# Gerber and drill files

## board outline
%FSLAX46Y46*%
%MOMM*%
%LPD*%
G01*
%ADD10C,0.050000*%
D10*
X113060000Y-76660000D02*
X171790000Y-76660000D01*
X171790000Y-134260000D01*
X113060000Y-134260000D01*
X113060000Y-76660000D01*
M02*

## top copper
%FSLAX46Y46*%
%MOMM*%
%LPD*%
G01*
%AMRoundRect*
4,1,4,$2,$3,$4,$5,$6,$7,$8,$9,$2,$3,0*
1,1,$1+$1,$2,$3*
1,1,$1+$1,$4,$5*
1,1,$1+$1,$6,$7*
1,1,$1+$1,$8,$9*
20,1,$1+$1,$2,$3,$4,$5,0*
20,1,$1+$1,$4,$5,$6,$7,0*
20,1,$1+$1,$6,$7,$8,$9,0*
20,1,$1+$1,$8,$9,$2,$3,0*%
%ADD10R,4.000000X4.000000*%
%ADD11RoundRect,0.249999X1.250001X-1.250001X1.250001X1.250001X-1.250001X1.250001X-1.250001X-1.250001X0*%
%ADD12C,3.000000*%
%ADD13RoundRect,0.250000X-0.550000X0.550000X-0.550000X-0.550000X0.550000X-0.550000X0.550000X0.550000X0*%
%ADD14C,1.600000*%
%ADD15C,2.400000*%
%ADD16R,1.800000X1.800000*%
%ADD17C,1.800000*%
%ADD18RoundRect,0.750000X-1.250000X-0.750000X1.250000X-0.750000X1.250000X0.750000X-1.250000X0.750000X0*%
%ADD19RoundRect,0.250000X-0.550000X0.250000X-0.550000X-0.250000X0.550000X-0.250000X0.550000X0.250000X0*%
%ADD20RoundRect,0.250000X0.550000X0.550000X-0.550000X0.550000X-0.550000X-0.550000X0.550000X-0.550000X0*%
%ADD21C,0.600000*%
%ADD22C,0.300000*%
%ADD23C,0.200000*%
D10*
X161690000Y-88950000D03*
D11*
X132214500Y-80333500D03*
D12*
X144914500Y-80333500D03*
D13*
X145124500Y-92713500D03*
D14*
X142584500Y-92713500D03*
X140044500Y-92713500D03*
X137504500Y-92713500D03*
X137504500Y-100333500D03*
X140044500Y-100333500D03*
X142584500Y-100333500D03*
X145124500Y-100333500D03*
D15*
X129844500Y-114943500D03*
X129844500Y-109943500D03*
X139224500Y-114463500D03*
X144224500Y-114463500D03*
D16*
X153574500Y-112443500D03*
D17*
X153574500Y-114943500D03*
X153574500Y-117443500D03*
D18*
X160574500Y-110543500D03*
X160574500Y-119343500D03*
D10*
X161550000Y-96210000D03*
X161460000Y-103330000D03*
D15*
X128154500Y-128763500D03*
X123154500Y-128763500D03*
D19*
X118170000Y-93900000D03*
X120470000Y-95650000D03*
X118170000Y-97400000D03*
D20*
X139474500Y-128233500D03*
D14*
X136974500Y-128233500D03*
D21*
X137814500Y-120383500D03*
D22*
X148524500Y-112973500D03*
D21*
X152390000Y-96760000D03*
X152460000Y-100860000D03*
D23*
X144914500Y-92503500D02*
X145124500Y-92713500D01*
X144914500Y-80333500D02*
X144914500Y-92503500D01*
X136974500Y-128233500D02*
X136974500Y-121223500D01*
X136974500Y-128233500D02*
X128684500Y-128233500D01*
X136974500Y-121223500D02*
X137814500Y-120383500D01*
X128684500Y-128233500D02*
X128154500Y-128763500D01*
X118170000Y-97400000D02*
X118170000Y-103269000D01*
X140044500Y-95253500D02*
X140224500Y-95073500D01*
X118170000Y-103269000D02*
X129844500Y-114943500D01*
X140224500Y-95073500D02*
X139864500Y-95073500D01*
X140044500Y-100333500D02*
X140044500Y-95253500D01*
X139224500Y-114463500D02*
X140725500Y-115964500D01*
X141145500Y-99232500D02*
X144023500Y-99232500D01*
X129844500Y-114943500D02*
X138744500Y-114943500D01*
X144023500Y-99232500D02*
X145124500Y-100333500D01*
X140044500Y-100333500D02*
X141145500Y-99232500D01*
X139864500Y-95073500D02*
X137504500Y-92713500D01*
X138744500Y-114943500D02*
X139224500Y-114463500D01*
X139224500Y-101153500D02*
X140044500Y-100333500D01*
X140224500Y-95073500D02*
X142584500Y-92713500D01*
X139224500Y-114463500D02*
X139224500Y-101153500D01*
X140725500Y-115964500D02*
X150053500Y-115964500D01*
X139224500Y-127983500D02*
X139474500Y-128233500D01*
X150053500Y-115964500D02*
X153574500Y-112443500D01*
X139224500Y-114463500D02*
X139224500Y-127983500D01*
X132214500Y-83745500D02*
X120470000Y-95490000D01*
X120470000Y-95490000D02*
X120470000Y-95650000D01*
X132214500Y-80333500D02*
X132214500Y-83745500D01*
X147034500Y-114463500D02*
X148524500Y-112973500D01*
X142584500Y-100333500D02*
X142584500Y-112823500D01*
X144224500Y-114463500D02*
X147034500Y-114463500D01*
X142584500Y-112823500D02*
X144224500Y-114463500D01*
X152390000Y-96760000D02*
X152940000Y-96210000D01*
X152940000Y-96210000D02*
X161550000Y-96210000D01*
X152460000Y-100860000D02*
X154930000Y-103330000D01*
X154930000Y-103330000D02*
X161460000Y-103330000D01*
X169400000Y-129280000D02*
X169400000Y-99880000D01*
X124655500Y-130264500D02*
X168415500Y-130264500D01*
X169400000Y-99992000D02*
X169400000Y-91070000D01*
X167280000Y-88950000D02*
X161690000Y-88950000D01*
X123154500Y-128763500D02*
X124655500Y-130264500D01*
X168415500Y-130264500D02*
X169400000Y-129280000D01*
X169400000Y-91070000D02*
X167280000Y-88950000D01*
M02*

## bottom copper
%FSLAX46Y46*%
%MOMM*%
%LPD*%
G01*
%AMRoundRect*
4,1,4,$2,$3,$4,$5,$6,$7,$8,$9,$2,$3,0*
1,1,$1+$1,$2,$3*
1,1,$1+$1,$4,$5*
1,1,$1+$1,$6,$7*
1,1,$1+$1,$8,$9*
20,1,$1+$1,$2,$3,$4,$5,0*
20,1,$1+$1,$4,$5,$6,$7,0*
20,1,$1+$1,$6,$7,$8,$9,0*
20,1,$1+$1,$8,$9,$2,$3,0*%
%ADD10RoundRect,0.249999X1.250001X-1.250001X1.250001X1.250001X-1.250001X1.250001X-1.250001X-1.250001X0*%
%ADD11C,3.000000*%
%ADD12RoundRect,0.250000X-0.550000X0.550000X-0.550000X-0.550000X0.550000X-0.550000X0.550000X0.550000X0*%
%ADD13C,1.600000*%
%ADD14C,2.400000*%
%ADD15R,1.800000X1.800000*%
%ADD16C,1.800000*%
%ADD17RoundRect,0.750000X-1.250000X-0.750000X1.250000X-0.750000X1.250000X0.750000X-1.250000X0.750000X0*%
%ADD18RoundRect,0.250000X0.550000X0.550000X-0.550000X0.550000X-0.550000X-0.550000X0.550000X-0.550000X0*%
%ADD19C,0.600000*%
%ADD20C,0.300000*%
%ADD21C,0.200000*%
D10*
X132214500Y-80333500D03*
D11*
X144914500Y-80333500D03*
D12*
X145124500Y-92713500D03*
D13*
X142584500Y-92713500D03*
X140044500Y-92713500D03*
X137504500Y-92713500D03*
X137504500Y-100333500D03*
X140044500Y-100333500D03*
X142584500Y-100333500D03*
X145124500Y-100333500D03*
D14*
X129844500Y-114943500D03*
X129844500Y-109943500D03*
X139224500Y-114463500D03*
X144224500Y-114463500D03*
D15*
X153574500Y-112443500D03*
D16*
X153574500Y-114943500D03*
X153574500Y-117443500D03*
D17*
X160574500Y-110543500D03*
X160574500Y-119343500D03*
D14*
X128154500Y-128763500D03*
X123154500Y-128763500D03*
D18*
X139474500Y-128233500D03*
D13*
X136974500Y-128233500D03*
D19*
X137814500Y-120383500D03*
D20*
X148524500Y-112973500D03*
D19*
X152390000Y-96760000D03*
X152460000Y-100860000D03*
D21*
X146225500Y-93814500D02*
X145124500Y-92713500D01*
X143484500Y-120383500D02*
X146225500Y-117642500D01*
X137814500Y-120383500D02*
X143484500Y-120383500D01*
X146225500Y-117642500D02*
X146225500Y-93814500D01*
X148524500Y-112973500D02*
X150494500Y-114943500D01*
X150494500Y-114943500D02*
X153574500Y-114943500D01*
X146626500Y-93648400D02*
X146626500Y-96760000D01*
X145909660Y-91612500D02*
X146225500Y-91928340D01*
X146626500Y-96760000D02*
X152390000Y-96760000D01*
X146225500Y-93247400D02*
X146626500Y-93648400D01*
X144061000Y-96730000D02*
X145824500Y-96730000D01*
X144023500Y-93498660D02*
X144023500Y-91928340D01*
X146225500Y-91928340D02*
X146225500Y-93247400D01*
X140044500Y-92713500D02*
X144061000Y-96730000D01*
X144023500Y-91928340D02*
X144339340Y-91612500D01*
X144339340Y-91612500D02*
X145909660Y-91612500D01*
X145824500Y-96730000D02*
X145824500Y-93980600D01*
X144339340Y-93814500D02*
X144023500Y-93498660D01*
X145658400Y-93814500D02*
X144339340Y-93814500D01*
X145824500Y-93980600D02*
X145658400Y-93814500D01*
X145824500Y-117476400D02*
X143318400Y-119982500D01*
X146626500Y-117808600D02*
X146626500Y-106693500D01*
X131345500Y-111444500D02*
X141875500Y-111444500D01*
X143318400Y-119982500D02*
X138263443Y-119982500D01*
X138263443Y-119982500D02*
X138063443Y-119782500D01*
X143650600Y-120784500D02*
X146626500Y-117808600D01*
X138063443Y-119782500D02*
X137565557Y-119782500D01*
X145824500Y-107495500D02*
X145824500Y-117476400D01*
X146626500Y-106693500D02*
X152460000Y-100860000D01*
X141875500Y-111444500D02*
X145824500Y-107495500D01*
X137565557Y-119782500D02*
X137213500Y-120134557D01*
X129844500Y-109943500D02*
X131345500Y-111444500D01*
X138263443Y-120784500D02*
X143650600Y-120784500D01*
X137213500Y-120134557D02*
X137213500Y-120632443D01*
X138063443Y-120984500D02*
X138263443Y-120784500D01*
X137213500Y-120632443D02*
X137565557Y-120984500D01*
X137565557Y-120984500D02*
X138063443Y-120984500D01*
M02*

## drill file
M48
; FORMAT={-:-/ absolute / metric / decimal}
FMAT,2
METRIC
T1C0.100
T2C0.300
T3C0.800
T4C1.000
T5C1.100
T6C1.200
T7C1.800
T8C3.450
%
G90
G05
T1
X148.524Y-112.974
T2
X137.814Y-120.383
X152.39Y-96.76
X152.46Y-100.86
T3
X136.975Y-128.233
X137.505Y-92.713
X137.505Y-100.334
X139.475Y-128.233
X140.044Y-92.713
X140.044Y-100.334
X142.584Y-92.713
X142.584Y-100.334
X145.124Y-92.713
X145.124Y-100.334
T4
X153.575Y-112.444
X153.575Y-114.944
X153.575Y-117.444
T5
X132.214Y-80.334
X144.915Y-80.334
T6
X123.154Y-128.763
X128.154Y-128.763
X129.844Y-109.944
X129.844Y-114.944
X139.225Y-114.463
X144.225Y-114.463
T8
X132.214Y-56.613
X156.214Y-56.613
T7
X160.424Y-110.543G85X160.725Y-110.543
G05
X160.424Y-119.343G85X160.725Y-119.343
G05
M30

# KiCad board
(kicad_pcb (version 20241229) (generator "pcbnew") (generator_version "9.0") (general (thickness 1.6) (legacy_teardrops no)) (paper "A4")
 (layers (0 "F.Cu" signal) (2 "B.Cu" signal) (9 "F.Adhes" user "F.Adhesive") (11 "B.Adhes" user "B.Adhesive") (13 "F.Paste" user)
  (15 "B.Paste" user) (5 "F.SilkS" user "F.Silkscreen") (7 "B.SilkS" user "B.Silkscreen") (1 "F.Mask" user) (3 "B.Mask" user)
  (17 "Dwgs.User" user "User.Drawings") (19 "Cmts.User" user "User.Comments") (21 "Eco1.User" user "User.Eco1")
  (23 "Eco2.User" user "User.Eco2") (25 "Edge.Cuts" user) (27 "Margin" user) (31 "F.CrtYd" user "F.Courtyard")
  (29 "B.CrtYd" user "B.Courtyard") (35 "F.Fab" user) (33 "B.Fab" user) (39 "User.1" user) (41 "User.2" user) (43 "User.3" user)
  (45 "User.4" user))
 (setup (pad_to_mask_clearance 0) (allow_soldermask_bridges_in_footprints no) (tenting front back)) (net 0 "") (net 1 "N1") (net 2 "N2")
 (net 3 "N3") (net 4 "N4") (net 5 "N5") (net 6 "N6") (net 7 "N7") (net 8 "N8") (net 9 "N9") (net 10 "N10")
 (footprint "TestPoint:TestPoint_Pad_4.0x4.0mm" (layer "F.Cu") (at 161.69 88.95)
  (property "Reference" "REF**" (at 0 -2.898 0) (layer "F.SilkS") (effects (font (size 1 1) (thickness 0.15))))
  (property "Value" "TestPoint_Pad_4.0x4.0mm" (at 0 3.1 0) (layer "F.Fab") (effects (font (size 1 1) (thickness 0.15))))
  (pad "1" smd rect (at 0 0) (size 4 4) (layers "F.Cu" "F.Mask") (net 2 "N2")))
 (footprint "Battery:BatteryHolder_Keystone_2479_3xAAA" (layer "F.Cu") (at 132.2145 80.3335 90)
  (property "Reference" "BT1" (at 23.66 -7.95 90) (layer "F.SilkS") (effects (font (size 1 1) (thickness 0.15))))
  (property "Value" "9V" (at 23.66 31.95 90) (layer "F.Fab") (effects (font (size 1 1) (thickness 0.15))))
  (pad "" np_thru_hole circle (at 23.72 0 90) (size 3.45 3.45) (drill 3.45) (layers "*.Cu" "*.Mask"))
  (pad "" np_thru_hole circle (at 23.72 24 90) (size 3.45 3.45) (drill 3.45) (layers "*.Cu" "*.Mask"))
  (pad "1" thru_hole roundrect (at 0 0 90) (size 3 3) (drill 1.1) (layers "*.Cu" "*.Mask") (remove_unused_layers no)
   (roundrect_rratio 0.083333) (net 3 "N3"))
  (pad "2" thru_hole circle (at 0 12.7 90) (size 3 3) (drill 1.1) (layers "*.Cu" "*.Mask") (remove_unused_layers no) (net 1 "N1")))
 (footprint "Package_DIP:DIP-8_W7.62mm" (layer "F.Cu") (at 145.1245 92.7135 -90)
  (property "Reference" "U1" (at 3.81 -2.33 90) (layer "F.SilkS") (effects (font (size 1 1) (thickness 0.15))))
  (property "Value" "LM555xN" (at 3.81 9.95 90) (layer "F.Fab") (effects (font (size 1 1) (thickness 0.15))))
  (pad "1" thru_hole roundrect (at 0 0 270) (size 1.6 1.6) (drill 0.8) (layers "*.Cu" "*.Mask") (remove_unused_layers no)
   (roundrect_rratio 0.15625) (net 1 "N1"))
  (pad "2" thru_hole circle (at 0 2.54 270) (size 1.6 1.6) (drill 0.8) (layers "*.Cu" "*.Mask") (remove_unused_layers no) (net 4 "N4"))
  (pad "3" thru_hole circle (at 0 5.08 270) (size 1.6 1.6) (drill 0.8) (layers "*.Cu" "*.Mask") (remove_unused_layers no) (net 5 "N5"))
  (pad "4" thru_hole circle (at 0 7.62 270) (size 1.6 1.6) (drill 0.8) (layers "*.Cu" "*.Mask") (remove_unused_layers no) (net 4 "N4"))
  (pad "5" thru_hole circle (at 7.62 7.62 270) (size 1.6 1.6) (drill 0.8) (layers "*.Cu" "*.Mask") (remove_unused_layers no) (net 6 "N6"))
  (pad "6" thru_hole circle (at 7.62 5.08 270) (size 1.6 1.6) (drill 0.8) (layers "*.Cu" "*.Mask") (remove_unused_layers no) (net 4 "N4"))
  (pad "7" thru_hole circle (at 7.62 2.54 270) (size 1.6 1.6) (drill 0.8) (layers "*.Cu" "*.Mask") (remove_unused_layers no) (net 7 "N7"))
  (pad "8" thru_hole circle (at 7.62 0 270) (size 1.6 1.6) (drill 0.8) (layers "*.Cu" "*.Mask") (remove_unused_layers no) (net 4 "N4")))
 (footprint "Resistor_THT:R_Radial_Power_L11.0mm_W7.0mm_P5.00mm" (layer "F.Cu") (at 129.8445 114.9435 90)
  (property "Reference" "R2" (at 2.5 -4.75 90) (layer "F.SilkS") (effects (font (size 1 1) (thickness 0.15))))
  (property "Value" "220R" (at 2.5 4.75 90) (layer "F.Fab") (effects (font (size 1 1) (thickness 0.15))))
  (pad "1" thru_hole circle (at 0 0 90) (size 2.4 2.4) (drill 1.2) (layers "*.Cu" "*.Mask") (remove_unused_layers no) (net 4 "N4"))
  (pad "2" thru_hole circle (at 5 0 90) (size 2.4 2.4) (drill 1.2) (layers "*.Cu" "*.Mask") (remove_unused_layers no) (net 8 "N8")))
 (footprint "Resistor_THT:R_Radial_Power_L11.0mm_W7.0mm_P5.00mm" (layer "F.Cu") (at 139.2245 114.4635)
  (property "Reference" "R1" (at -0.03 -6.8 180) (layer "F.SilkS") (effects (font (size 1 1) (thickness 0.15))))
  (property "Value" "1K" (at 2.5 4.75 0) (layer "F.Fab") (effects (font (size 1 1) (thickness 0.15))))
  (pad "1" thru_hole circle (at 0 0) (size 2.4 2.4) (drill 1.2) (layers "*.Cu" "*.Mask") (remove_unused_layers no) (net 4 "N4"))
  (pad "2" thru_hole circle (at 5 0) (size 2.4 2.4) (drill 1.2) (layers "*.Cu" "*.Mask") (remove_unused_layers no) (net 7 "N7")))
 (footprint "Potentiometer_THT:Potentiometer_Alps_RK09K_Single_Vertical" (layer "F.Cu") (at 153.5745 112.4435)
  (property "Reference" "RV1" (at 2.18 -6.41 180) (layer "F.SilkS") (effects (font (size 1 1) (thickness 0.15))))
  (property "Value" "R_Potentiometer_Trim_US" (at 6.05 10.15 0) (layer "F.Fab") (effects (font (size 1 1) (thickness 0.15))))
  (pad "1" thru_hole rect (at 0 0) (size 1.8 1.8) (drill 1) (layers "*.Cu" "*.Mask") (remove_unused_layers no) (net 4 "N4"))
  (pad "2" thru_hole circle (at 0 2.5) (size 1.8 1.8) (drill 1) (layers "*.Cu" "*.Mask") (remove_unused_layers no) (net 7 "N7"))
  (pad "3" thru_hole circle (at 0 5) (size 1.8 1.8) (drill 1) (layers "*.Cu" "*.Mask") (remove_unused_layers no) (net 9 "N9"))
  (pad "MP" thru_hole roundrect (at 7 -1.9) (size 4 3) (drill oval 2.1 1.8) (layers "*.Cu" "*.Mask") (remove_unused_layers no)
   (roundrect_rratio 0.25))
  (pad "MP" thru_hole roundrect (at 7 6.9) (size 4 3) (drill oval 2.1 1.8) (layers "*.Cu" "*.Mask") (remove_unused_layers no)
   (roundrect_rratio 0.25)))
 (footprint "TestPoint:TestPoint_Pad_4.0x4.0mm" (layer "F.Cu") (at 161.55 96.21)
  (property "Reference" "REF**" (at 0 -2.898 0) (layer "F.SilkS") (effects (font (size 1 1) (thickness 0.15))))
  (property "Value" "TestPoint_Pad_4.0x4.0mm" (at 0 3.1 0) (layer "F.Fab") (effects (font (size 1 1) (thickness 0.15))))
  (pad "1" smd rect (at 0 0) (size 4 4) (layers "F.Cu" "F.Mask") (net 5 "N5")))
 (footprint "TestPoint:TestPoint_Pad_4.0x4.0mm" (layer "F.Cu") (at 161.46 103.33)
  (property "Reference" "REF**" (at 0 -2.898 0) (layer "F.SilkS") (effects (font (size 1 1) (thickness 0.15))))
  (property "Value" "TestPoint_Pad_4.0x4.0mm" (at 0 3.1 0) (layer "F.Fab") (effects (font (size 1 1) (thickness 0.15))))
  (pad "1" smd rect (at 0 0) (size 4 4) (layers "F.Cu" "F.Mask") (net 8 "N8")))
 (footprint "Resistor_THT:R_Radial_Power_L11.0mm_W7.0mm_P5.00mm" (layer "F.Cu") (at 128.1545 128.7635 180)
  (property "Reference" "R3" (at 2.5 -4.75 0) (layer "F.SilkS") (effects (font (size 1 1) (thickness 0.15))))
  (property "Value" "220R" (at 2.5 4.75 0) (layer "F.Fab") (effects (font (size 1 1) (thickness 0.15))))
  (pad "1" thru_hole circle (at 0 0 180) (size 2.4 2.4) (drill 1.2) (layers "*.Cu" "*.Mask") (remove_unused_layers no) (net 1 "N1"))
  (pad "2" thru_hole circle (at 5 0 180) (size 2.4 2.4) (drill 1.2) (layers "*.Cu" "*.Mask") (remove_unused_layers no) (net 2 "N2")))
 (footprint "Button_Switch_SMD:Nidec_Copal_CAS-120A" (layer "F.Cu") (at 119.32 95.65)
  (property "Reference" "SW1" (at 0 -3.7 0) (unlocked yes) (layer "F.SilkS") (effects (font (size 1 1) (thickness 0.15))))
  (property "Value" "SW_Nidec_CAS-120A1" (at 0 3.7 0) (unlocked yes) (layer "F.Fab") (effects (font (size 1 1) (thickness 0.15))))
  (pad "1" smd roundrect (at -1.15 -1.75 270) (size 1 1.6) (layers "F.Cu" "F.Mask" "F.Paste") (roundrect_rratio 0.25) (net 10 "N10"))
  (pad "2" smd roundrect (at 1.15 0 270) (size 1 1.6) (layers "F.Cu" "F.Mask" "F.Paste") (roundrect_rratio 0.25) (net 3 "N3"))
  (pad "3" smd roundrect (at -1.15 1.75 270) (size 1 1.6) (layers "F.Cu" "F.Mask" "F.Paste") (roundrect_rratio 0.25) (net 4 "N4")))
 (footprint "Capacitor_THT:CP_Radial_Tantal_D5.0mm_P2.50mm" (layer "F.Cu") (at 139.4745 128.2335 180)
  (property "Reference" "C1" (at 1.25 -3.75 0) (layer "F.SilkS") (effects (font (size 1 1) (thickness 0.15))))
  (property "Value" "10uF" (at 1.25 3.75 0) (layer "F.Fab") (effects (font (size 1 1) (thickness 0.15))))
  (pad "1" thru_hole roundrect (at 0 0 180) (size 1.6 1.6) (drill 0.8) (layers "*.Cu" "*.Mask") (remove_unused_layers no)
   (roundrect_rratio 0.15625) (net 4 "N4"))
  (pad "2" thru_hole circle (at 2.5 0 180) (size 1.6 1.6) (drill 0.8) (layers "*.Cu" "*.Mask") (remove_unused_layers no) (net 1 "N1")))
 (gr_rect (start 113.06 76.66) (end 171.79 134.26) (stroke (width 0.05) (type default)) (fill no) (layer "Edge.Cuts"))
 (segment (start 144.9145 92.5035) (end 145.1245 92.7135) (width 0.2) (layer "F.Cu") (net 1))
 (segment (start 144.9145 80.3335) (end 144.9145 92.5035) (width 0.2) (layer "F.Cu") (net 1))
 (segment (start 136.9745 128.2335) (end 136.9745 121.2235) (width 0.2) (layer "F.Cu") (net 1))
 (segment (start 136.9745 128.2335) (end 128.6845 128.2335) (width 0.2) (layer "F.Cu") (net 1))
 (segment (start 136.9745 121.2235) (end 137.8145 120.3835) (width 0.2) (layer "F.Cu") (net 1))
 (segment (start 128.6845 128.2335) (end 128.1545 128.7635) (width 0.2) (layer "F.Cu") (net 1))
 (via (at 137.8145 120.3835) (size 0.6) (drill 0.3) (layers "F.Cu" "B.Cu") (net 1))
 (segment (start 146.2255 93.8145) (end 145.1245 92.7135) (width 0.2) (layer "B.Cu") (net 1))
 (segment (start 143.4845 120.3835) (end 146.2255 117.6425) (width 0.2) (layer "B.Cu") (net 1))
 (segment (start 137.8145 120.3835) (end 143.4845 120.3835) (width 0.2) (layer "B.Cu") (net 1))
 (segment (start 146.2255 117.6425) (end 146.2255 93.8145) (width 0.2) (layer "B.Cu") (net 1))
 (segment (start 118.17 97.4) (end 118.17 103.269) (width 0.2) (layer "F.Cu") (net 4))
 (segment (start 140.0445 95.2535) (end 140.2245 95.0735) (width 0.2) (layer "F.Cu") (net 4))
 (segment (start 118.17 103.269) (end 129.8445 114.9435) (width 0.2) (layer "F.Cu") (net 4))
 (segment (start 140.2245 95.0735) (end 139.8645 95.0735) (width 0.2) (layer "F.Cu") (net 4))
 (segment (start 140.0445 100.3335) (end 140.0445 95.2535) (width 0.2) (layer "F.Cu") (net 4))
 (segment (start 139.2245 114.4635) (end 140.7255 115.9645) (width 0.2) (layer "F.Cu") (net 4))
 (segment (start 141.1455 99.2325) (end 144.0235 99.2325) (width 0.2) (layer "F.Cu") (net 4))
 (segment (start 129.8445 114.9435) (end 138.7445 114.9435) (width 0.2) (layer "F.Cu") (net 4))
 (segment (start 144.0235 99.2325) (end 145.1245 100.3335) (width 0.2) (layer "F.Cu") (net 4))
 (segment (start 140.0445 100.3335) (end 141.1455 99.2325) (width 0.2) (layer "F.Cu") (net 4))
 (segment (start 139.8645 95.0735) (end 137.5045 92.7135) (width 0.2) (layer "F.Cu") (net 4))
 (segment (start 138.7445 114.9435) (end 139.2245 114.4635) (width 0.2) (layer "F.Cu") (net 4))
 (segment (start 139.2245 101.1535) (end 140.0445 100.3335) (width 0.2) (layer "F.Cu") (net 4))
 (segment (start 140.2245 95.0735) (end 142.5845 92.7135) (width 0.2) (layer "F.Cu") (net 4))
 (segment (start 139.2245 114.4635) (end 139.2245 101.1535) (width 0.2) (layer "F.Cu") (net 4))
 (segment (start 140.7255 115.9645) (end 150.0535 115.9645) (width 0.2) (layer "F.Cu") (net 4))
 (segment (start 139.2245 127.9835) (end 139.4745 128.2335) (width 0.2) (layer "F.Cu") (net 4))
 (segment (start 150.0535 115.9645) (end 153.5745 112.4435) (width 0.2) (layer "F.Cu") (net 4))
 (segment (start 139.2245 114.4635) (end 139.2245 127.9835) (width 0.2) (layer "F.Cu") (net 4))
 (segment (start 132.2145 83.7455) (end 120.47 95.49) (width 0.2) (layer "F.Cu") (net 3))
 (segment (start 120.47 95.49) (end 120.47 95.65) (width 0.2) (layer "F.Cu") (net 3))
 (segment (start 132.2145 80.3335) (end 132.2145 83.7455) (width 0.2) (layer "F.Cu") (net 3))
 (segment (start 147.0345 114.4635) (end 148.5245 112.9735) (width 0.2) (layer "F.Cu") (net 7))
 (segment (start 142.5845 100.3335) (end 142.5845 112.8235) (width 0.2) (layer "F.Cu") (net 7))
 (segment (start 144.2245 114.4635) (end 147.0345 114.4635) (width 0.2) (layer "F.Cu") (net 7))
 (segment (start 142.5845 112.8235) (end 144.2245 114.4635) (width 0.2) (layer "F.Cu") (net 7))
 (via micro (at 148.5245 112.9735) (size 0.3) (drill 0.1) (layers "F.Cu" "B.Cu") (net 7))
 (segment (start 148.5245 112.9735) (end 150.4945 114.9435) (width 0.2) (layer "B.Cu") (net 7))
 (segment (start 150.4945 114.9435) (end 153.5745 114.9435) (width 0.2) (layer "B.Cu") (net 7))
 (segment (start 152.39 96.76) (end 152.94 96.21) (width 0.2) (layer "F.Cu") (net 5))
 (segment (start 152.94 96.21) (end 161.55 96.21) (width 0.2) (layer "F.Cu") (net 5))
 (via (at 152.39 96.76) (size 0.6) (drill 0.3) (layers "F.Cu" "B.Cu") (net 5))
 (segment (start 146.6265 93.6484) (end 146.6265 96.76) (width 0.2) (layer "B.Cu") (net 5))
 (segment (start 145.90966 91.6125) (end 146.2255 91.92834) (width 0.2) (layer "B.Cu") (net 5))
 (segment (start 146.6265 96.76) (end 152.39 96.76) (width 0.2) (layer "B.Cu") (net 5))
 (segment (start 146.2255 93.2474) (end 146.6265 93.6484) (width 0.2) (layer "B.Cu") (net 5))
 (segment (start 144.061 96.73) (end 145.8245 96.73) (width 0.2) (layer "B.Cu") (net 5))
 (segment (start 144.0235 93.49866) (end 144.0235 91.92834) (width 0.2) (layer "B.Cu") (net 5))
 (segment (start 146.2255 91.92834) (end 146.2255 93.2474) (width 0.2) (layer "B.Cu") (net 5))
 (segment (start 140.0445 92.7135) (end 144.061 96.73) (width 0.2) (layer "B.Cu") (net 5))
 (segment (start 144.0235 91.92834) (end 144.33934 91.6125) (width 0.2) (layer "B.Cu") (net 5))
 (segment (start 144.33934 91.6125) (end 145.90966 91.6125) (width 0.2) (layer "B.Cu") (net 5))
 (segment (start 145.8245 96.73) (end 145.8245 93.9806) (width 0.2) (layer "B.Cu") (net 5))
 (segment (start 144.33934 93.8145) (end 144.0235 93.49866) (width 0.2) (layer "B.Cu") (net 5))
 (segment (start 145.6584 93.8145) (end 144.33934 93.8145) (width 0.2) (layer "B.Cu") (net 5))
 (segment (start 145.8245 93.9806) (end 145.6584 93.8145) (width 0.2) (layer "B.Cu") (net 5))
 (segment (start 152.46 100.86) (end 154.93 103.33) (width 0.2) (layer "F.Cu") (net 8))
 (segment (start 154.93 103.33) (end 161.46 103.33) (width 0.2) (layer "F.Cu") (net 8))
 (via (at 152.46 100.86) (size 0.6) (drill 0.3) (layers "F.Cu" "B.Cu") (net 8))
 (segment (start 145.8245 117.4764) (end 143.3184 119.9825) (width 0.2) (layer "B.Cu") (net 8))
 (segment (start 146.6265 117.8086) (end 146.6265 106.6935) (width 0.2) (layer "B.Cu") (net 8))
 (segment (start 131.3455 111.4445) (end 141.8755 111.4445) (width 0.2) (layer "B.Cu") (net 8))
 (segment (start 143.3184 119.9825) (end 138.263443 119.9825) (width 0.2) (layer "B.Cu") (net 8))
 (segment (start 138.263443 119.9825) (end 138.063443 119.7825) (width 0.2) (layer "B.Cu") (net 8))
 (segment (start 143.6506 120.7845) (end 146.6265 117.8086) (width 0.2) (layer "B.Cu") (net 8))
 (segment (start 138.063443 119.7825) (end 137.565557 119.7825) (width 0.2) (layer "B.Cu") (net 8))
 (segment (start 145.8245 107.4955) (end 145.8245 117.4764) (width 0.2) (layer "B.Cu") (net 8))
 (segment (start 146.6265 106.6935) (end 152.46 100.86) (width 0.2) (layer "B.Cu") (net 8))
 (segment (start 141.8755 111.4445) (end 145.8245 107.4955) (width 0.2) (layer "B.Cu") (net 8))
 (segment (start 137.565557 119.7825) (end 137.2135 120.134557) (width 0.2) (layer "B.Cu") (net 8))
 (segment (start 129.8445 109.9435) (end 131.3455 111.4445) (width 0.2) (layer "B.Cu") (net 8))
 (segment (start 138.263443 120.7845) (end 143.6506 120.7845) (width 0.2) (layer "B.Cu") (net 8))
 (segment (start 137.2135 120.134557) (end 137.2135 120.632443) (width 0.2) (layer "B.Cu") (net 8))
 (segment (start 138.063443 120.9845) (end 138.263443 120.7845) (width 0.2) (layer "B.Cu") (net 8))
 (segment (start 137.2135 120.632443) (end 137.565557 120.9845) (width 0.2) (layer "B.Cu") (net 8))
 (segment (start 137.565557 120.9845) (end 138.063443 120.9845) (width 0.2) (layer "B.Cu") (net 8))
 (segment (start 169.4 129.28) (end 169.4 99.88) (width 0.2) (layer "F.Cu") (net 2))
 (segment (start 124.6555 130.2645) (end 168.4155 130.2645) (width 0.2) (layer "F.Cu") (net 2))
 (segment (start 169.4 99.992) (end 169.4 91.07) (width 0.2) (layer "F.Cu") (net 2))
 (segment (start 167.28 88.95) (end 161.69 88.95) (width 0.2) (layer "F.Cu") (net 2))
 (segment (start 123.1545 128.7635) (end 124.6555 130.2645) (width 0.2) (layer "F.Cu") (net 2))
 (segment (start 168.4155 130.2645) (end 169.4 129.28) (width 0.2) (layer "F.Cu") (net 2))
 (segment (start 169.4 91.07) (end 167.28 88.95) (width 0.2) (layer "F.Cu") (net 2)))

